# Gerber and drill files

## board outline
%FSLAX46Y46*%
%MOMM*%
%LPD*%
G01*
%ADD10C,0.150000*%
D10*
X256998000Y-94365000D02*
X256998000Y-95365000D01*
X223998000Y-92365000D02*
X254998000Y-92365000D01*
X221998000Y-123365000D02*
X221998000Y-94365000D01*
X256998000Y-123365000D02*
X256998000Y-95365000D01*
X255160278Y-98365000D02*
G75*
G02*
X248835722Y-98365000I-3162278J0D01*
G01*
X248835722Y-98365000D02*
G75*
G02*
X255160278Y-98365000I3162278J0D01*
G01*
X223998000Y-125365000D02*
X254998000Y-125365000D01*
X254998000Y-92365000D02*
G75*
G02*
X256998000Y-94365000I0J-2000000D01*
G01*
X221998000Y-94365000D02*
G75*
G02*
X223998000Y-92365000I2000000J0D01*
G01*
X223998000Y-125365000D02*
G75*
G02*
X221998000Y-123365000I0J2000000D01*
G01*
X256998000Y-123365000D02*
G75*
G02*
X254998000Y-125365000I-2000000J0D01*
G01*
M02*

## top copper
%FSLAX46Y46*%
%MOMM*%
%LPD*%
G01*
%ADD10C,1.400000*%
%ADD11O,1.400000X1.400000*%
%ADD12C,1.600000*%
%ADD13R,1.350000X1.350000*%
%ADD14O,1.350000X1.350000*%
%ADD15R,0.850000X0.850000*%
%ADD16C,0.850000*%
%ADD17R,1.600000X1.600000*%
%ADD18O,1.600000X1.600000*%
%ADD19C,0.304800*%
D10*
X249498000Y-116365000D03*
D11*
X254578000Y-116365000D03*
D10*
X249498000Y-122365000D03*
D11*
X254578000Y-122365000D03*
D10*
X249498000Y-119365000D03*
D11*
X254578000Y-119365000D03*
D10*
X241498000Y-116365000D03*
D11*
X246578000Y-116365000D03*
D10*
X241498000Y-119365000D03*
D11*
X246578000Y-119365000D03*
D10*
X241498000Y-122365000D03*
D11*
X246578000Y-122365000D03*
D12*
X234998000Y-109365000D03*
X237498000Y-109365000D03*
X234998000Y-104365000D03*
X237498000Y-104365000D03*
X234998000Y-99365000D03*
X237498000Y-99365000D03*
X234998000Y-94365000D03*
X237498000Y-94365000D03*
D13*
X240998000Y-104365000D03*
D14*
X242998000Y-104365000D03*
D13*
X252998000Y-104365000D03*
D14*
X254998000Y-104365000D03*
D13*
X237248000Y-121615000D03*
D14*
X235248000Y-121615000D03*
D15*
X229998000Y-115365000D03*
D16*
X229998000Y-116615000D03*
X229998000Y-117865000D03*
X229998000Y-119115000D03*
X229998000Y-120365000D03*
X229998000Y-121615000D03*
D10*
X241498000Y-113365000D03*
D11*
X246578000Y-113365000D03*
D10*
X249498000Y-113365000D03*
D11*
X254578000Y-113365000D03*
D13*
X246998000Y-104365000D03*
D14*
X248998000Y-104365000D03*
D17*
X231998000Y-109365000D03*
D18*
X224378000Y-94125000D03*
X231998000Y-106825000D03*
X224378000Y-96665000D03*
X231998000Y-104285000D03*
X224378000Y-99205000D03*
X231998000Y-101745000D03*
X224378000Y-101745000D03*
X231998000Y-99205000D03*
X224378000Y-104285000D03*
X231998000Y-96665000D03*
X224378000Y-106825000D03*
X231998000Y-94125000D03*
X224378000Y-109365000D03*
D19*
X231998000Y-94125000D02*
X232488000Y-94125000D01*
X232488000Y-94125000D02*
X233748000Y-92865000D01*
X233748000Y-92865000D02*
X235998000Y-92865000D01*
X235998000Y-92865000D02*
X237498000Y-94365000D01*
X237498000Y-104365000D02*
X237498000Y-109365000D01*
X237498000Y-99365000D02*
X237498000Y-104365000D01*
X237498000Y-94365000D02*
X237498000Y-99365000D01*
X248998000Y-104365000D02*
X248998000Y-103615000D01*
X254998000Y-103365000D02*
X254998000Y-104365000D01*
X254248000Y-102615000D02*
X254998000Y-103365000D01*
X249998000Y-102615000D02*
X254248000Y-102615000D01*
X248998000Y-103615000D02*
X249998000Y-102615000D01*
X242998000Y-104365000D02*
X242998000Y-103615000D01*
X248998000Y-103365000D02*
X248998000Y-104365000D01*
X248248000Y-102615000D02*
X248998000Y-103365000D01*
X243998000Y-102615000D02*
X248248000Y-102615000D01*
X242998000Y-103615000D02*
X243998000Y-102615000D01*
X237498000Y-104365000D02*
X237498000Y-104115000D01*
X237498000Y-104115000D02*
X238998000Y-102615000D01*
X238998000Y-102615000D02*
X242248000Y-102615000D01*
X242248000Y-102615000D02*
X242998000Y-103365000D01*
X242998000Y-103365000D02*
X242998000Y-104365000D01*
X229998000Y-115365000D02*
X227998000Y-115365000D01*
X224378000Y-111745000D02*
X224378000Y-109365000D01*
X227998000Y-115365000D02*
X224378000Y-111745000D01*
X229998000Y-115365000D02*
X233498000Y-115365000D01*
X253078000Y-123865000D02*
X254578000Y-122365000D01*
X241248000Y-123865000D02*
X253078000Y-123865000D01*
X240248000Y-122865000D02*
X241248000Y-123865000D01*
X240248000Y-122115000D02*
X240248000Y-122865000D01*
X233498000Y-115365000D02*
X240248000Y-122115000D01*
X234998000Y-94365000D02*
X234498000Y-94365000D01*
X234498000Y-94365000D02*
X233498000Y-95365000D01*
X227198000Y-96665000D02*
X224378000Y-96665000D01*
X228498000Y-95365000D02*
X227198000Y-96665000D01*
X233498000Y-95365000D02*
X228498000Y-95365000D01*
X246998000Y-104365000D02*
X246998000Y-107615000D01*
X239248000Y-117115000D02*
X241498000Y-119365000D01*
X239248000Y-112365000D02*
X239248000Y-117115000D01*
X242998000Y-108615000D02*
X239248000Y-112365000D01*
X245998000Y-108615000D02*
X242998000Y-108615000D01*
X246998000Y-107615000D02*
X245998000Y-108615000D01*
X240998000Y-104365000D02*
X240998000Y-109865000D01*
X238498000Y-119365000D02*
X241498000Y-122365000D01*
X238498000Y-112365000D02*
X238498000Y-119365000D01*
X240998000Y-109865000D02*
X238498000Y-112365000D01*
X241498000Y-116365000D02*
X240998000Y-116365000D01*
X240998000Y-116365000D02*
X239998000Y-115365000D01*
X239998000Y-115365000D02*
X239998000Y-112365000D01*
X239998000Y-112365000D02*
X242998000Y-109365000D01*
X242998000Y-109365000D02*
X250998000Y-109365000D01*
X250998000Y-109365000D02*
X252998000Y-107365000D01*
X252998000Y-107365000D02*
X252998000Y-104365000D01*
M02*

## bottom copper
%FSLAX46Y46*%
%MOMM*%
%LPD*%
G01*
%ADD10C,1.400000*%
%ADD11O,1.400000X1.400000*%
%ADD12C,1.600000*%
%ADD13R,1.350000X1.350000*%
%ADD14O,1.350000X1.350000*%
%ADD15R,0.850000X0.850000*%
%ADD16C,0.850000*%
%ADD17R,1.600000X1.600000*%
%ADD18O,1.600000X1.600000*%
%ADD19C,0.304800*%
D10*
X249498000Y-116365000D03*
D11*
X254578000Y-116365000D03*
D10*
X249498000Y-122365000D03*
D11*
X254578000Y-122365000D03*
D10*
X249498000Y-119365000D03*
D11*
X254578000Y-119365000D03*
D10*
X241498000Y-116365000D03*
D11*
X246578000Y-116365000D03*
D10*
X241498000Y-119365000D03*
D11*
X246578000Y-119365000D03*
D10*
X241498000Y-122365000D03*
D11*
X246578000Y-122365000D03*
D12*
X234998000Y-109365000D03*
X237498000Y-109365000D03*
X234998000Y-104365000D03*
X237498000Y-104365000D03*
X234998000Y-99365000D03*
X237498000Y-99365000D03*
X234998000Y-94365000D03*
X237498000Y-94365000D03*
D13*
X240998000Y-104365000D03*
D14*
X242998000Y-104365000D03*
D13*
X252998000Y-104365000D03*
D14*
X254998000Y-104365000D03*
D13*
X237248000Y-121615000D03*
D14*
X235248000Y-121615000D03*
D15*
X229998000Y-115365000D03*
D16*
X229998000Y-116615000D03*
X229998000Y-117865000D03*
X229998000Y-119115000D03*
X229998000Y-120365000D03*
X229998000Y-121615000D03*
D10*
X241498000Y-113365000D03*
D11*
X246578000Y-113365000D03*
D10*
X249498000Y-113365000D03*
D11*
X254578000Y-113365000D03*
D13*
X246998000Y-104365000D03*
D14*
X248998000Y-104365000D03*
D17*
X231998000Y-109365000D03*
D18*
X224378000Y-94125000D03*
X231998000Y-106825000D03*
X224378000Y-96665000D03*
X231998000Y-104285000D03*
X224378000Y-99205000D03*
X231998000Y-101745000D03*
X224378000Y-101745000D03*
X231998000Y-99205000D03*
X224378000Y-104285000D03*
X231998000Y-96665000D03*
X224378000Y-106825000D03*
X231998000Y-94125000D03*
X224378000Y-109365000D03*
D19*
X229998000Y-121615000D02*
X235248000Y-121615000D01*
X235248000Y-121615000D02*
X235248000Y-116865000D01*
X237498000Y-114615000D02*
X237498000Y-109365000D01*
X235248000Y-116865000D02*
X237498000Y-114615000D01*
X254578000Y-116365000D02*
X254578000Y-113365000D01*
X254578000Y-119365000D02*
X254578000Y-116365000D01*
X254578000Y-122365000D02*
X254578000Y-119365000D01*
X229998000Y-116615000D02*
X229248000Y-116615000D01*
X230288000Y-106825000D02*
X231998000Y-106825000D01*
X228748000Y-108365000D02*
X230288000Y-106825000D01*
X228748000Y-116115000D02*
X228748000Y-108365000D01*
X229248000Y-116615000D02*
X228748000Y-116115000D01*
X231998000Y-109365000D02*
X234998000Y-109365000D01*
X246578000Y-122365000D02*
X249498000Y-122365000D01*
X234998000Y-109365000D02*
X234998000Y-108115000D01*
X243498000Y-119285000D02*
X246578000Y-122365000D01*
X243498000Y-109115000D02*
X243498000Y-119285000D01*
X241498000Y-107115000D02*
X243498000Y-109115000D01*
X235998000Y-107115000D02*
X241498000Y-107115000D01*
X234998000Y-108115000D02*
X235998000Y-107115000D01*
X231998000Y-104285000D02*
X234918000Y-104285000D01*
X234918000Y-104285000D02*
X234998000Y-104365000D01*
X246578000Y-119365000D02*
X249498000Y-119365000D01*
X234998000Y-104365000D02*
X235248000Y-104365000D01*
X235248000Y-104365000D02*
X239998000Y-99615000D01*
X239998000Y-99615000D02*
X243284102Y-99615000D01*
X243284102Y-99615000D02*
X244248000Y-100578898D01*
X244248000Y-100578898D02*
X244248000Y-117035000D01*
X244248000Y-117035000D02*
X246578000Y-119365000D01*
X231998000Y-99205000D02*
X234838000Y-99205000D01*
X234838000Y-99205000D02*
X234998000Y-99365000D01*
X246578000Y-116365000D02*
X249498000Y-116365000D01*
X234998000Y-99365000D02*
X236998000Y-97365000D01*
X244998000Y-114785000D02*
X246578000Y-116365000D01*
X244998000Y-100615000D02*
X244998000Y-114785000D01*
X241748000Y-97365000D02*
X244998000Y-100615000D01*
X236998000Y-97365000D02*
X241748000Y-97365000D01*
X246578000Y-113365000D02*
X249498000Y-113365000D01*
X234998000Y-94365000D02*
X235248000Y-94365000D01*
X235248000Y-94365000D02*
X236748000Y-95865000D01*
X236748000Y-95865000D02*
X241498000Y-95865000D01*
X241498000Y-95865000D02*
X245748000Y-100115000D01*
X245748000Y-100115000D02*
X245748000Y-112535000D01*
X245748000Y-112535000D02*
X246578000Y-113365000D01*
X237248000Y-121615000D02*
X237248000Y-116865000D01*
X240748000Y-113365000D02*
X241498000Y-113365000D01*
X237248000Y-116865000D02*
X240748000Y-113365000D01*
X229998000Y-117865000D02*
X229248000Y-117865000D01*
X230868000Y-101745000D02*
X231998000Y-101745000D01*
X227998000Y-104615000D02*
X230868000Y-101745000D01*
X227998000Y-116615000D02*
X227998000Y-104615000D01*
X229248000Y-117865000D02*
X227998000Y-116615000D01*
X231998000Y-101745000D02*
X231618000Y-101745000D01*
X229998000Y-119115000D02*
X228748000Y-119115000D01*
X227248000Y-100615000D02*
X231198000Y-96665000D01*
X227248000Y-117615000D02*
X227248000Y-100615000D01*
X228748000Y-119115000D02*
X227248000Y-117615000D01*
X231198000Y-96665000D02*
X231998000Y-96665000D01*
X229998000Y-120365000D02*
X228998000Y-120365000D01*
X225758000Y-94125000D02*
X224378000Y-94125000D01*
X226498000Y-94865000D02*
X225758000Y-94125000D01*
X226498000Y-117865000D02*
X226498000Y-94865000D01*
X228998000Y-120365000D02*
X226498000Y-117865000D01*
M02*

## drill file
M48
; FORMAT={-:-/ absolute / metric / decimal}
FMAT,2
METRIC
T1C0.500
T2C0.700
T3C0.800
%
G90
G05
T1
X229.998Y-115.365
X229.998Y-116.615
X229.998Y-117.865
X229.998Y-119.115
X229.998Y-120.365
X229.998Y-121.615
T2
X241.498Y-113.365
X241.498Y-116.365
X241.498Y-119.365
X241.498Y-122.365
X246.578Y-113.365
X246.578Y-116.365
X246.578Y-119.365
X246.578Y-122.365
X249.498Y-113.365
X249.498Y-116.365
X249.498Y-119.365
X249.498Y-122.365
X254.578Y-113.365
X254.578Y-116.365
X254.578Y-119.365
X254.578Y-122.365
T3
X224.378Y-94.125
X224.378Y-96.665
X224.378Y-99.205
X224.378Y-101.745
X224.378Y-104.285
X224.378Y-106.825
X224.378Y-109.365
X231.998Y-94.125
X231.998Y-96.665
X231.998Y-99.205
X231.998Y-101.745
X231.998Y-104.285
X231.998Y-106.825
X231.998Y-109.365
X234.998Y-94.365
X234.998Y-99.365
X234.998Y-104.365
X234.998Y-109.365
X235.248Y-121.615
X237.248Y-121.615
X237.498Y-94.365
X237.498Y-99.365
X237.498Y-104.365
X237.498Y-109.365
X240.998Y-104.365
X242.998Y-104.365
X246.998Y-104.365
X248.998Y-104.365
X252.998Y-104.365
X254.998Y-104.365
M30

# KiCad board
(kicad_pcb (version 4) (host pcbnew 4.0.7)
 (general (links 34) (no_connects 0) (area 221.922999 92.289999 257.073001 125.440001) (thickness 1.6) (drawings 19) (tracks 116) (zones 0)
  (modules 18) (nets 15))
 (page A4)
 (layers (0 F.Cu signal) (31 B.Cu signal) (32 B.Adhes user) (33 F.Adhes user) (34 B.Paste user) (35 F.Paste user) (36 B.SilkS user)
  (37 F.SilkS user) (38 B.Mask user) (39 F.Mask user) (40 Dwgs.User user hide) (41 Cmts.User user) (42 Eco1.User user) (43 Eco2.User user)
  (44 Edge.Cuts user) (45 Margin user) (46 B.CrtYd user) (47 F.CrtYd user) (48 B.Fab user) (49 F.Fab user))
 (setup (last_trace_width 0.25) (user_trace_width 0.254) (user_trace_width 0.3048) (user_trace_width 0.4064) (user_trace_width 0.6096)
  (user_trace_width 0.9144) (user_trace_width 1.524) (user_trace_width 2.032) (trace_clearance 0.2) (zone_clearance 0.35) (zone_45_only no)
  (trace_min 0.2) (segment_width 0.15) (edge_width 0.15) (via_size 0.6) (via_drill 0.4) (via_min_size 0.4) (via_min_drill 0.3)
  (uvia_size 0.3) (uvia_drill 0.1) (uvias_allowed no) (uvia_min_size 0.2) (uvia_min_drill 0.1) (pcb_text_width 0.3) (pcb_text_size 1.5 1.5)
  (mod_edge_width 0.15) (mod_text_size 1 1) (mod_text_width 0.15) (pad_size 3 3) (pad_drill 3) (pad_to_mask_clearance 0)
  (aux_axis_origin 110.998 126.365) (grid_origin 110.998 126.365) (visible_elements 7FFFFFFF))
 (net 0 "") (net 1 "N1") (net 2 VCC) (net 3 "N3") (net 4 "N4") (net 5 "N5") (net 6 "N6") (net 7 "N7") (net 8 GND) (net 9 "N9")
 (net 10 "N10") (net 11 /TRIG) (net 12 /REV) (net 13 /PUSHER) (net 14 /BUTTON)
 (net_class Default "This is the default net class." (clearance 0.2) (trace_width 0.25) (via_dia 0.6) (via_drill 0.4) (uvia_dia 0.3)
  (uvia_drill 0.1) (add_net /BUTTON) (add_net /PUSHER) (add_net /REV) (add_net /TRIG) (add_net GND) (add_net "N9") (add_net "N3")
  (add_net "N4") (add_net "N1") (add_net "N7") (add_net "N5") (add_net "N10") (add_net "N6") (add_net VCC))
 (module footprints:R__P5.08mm (layer F.Cu) (at 251.998 116.365)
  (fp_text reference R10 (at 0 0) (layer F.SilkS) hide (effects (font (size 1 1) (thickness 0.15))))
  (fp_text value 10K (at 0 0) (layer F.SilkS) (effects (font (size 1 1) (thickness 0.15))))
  (pad 1 thru_hole circle (at -2.5 0) (size 1.4 1.4) (drill 0.7) (layers *.Cu *.Mask) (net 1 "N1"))
  (pad 2 thru_hole oval (at 2.58 0) (size 1.4 1.4) (drill 0.7) (layers *.Cu *.Mask) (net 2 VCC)))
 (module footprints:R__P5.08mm (layer F.Cu) (at 251.998 122.365)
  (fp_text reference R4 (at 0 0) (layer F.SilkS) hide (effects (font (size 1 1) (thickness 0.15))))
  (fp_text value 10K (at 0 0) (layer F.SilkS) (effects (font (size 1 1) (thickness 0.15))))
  (pad 1 thru_hole circle (at -2.5 0) (size 1.4 1.4) (drill 0.7) (layers *.Cu *.Mask) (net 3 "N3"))
  (pad 2 thru_hole oval (at 2.58 0) (size 1.4 1.4) (drill 0.7) (layers *.Cu *.Mask) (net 2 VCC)))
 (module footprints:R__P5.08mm (layer F.Cu) (at 251.998 119.365)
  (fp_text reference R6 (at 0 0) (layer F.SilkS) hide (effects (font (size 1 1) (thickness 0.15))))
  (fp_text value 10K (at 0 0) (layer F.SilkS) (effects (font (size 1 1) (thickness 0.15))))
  (pad 1 thru_hole circle (at -2.5 0) (size 1.4 1.4) (drill 0.7) (layers *.Cu *.Mask) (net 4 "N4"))
  (pad 2 thru_hole oval (at 2.58 0) (size 1.4 1.4) (drill 0.7) (layers *.Cu *.Mask) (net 2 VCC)))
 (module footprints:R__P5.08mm (layer F.Cu) (at 243.998 116.365)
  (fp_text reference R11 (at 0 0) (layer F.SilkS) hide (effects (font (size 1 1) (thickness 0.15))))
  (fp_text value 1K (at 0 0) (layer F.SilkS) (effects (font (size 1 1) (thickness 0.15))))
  (pad 1 thru_hole circle (at -2.5 0) (size 1.4 1.4) (drill 0.7) (layers *.Cu *.Mask) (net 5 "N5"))
  (pad 2 thru_hole oval (at 2.58 0) (size 1.4 1.4) (drill 0.7) (layers *.Cu *.Mask) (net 1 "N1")))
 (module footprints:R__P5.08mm (layer F.Cu) (at 243.998 119.365)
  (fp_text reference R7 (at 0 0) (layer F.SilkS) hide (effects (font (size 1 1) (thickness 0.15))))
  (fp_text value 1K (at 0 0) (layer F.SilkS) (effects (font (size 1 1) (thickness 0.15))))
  (pad 1 thru_hole circle (at -2.5 0) (size 1.4 1.4) (drill 0.7) (layers *.Cu *.Mask) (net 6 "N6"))
  (pad 2 thru_hole oval (at 2.58 0) (size 1.4 1.4) (drill 0.7) (layers *.Cu *.Mask) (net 4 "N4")))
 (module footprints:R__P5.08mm (layer F.Cu) (at 243.998 122.365)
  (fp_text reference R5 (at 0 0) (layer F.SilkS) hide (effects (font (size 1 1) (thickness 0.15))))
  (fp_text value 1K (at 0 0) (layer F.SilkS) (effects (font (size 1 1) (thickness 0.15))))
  (pad 1 thru_hole circle (at -2.5 0) (size 1.4 1.4) (drill 0.7) (layers *.Cu *.Mask) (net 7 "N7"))
  (pad 2 thru_hole oval (at 2.58 0) (size 1.4 1.4) (drill 0.7) (layers *.Cu *.Mask) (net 3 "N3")))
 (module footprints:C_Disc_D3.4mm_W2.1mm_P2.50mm (layer F.Cu) (at 234.998 109.365)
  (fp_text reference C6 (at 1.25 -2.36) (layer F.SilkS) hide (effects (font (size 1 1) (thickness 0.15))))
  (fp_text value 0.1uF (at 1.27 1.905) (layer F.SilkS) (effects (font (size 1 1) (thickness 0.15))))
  (pad 1 thru_hole circle (at 0 0) (size 1.6 1.6) (drill 0.8) (layers *.Cu *.Mask) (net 3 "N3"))
  (pad 2 thru_hole circle (at 2.5 0) (size 1.6 1.6) (drill 0.8) (layers *.Cu *.Mask) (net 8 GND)))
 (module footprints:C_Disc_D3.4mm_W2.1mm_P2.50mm (layer F.Cu) (at 234.998 104.365)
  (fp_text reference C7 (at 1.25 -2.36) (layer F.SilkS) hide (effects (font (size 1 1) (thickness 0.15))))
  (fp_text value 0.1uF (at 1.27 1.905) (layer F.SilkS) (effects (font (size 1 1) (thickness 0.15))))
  (pad 1 thru_hole circle (at 0 0) (size 1.6 1.6) (drill 0.8) (layers *.Cu *.Mask) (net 4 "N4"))
  (pad 2 thru_hole circle (at 2.5 0) (size 1.6 1.6) (drill 0.8) (layers *.Cu *.Mask) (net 8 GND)))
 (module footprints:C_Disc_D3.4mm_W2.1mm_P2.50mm (layer F.Cu) (at 234.998 99.365)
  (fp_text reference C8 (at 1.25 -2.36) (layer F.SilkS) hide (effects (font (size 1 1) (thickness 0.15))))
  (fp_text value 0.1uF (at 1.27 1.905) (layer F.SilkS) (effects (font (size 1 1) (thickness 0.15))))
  (pad 1 thru_hole circle (at 0 0) (size 1.6 1.6) (drill 0.8) (layers *.Cu *.Mask) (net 1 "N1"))
  (pad 2 thru_hole circle (at 2.5 0) (size 1.6 1.6) (drill 0.8) (layers *.Cu *.Mask) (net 8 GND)))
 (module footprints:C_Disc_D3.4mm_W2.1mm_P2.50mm (layer F.Cu) (at 234.998 94.365)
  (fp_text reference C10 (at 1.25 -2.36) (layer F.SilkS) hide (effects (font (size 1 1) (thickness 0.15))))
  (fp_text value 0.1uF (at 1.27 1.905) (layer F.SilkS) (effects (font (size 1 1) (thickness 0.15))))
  (pad 1 thru_hole circle (at 0 0) (size 1.6 1.6) (drill 0.8) (layers *.Cu *.Mask) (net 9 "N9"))
  (pad 2 thru_hole circle (at 2.5 0) (size 1.6 1.6) (drill 0.8) (layers *.Cu *.Mask) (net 8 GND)))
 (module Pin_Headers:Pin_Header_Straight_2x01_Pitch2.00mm (layer F.Cu) (at 240.998 104.365)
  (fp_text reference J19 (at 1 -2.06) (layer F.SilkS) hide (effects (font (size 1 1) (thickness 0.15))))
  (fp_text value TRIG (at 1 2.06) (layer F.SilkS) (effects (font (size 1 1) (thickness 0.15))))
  (pad 1 thru_hole rect (at 0 0) (size 1.35 1.35) (drill 0.8) (layers *.Cu *.Mask) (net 7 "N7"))
  (pad 2 thru_hole oval (at 2 0) (size 1.35 1.35) (drill 0.8) (layers *.Cu *.Mask) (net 8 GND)))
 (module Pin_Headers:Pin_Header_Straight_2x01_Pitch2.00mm (layer F.Cu) (at 252.998 104.365)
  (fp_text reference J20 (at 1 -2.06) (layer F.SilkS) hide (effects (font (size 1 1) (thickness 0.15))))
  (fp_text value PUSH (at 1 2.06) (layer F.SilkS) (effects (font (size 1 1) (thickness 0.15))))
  (pad 1 thru_hole rect (at 0 0) (size 1.35 1.35) (drill 0.8) (layers *.Cu *.Mask) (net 5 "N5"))
  (pad 2 thru_hole oval (at 2 0) (size 1.35 1.35) (drill 0.8) (layers *.Cu *.Mask) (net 8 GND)))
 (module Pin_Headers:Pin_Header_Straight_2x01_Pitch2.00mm (layer F.Cu) (at 237.248 121.615 180)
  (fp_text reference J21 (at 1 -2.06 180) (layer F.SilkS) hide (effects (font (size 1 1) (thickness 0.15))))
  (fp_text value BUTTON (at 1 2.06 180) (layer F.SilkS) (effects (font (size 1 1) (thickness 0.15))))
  (pad 1 thru_hole rect (at 0 0 180) (size 1.35 1.35) (drill 0.8) (layers *.Cu *.Mask) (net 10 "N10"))
  (pad 2 thru_hole oval (at 2 0 180) (size 1.35 1.35) (drill 0.8) (layers *.Cu *.Mask) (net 8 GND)))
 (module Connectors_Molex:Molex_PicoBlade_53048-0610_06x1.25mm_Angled (layer F.Cu) (at 229.998 115.365 270)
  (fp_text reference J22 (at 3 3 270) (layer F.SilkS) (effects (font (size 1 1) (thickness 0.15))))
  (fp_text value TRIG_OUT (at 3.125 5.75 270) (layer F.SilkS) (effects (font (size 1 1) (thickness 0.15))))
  (pad 1 thru_hole rect (at 0 0 270) (size 0.85 0.85) (drill 0.5) (layers *.Cu *.Mask) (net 2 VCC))
  (pad 2 thru_hole circle (at 1.25 0 270) (size 0.85 0.85) (drill 0.5) (layers *.Cu *.Mask) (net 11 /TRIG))
  (pad 3 thru_hole circle (at 2.5 0 270) (size 0.85 0.85) (drill 0.5) (layers *.Cu *.Mask) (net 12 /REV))
  (pad 4 thru_hole circle (at 3.75 0 270) (size 0.85 0.85) (drill 0.5) (layers *.Cu *.Mask) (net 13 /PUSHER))
  (pad 5 thru_hole circle (at 5 0 270) (size 0.85 0.85) (drill 0.5) (layers *.Cu *.Mask) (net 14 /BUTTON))
  (pad 6 thru_hole circle (at 6.25 0 270) (size 0.85 0.85) (drill 0.5) (layers *.Cu *.Mask) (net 8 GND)))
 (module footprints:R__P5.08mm (layer F.Cu) (at 243.998 113.365)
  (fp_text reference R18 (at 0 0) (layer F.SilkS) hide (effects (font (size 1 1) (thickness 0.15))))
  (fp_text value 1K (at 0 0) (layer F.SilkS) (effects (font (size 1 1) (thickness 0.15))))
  (pad 1 thru_hole circle (at -2.5 0) (size 1.4 1.4) (drill 0.7) (layers *.Cu *.Mask) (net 10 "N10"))
  (pad 2 thru_hole oval (at 2.58 0) (size 1.4 1.4) (drill 0.7) (layers *.Cu *.Mask) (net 9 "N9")))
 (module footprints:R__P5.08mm (layer F.Cu) (at 251.998 113.365)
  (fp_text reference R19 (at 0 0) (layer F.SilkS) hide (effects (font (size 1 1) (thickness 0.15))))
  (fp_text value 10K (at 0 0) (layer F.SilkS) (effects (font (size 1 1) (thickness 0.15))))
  (pad 1 thru_hole circle (at -2.5 0) (size 1.4 1.4) (drill 0.7) (layers *.Cu *.Mask) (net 9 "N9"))
  (pad 2 thru_hole oval (at 2.58 0) (size 1.4 1.4) (drill 0.7) (layers *.Cu *.Mask) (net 2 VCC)))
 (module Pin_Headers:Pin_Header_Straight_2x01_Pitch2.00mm (layer F.Cu) (at 246.998 104.365)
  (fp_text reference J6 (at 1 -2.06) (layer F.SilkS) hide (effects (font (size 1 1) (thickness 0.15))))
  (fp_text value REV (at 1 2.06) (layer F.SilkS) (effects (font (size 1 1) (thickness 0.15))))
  (pad 1 thru_hole rect (at 0 0) (size 1.35 1.35) (drill 0.8) (layers *.Cu *.Mask) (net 6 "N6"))
  (pad 2 thru_hole oval (at 2 0) (size 1.35 1.35) (drill 0.8) (layers *.Cu *.Mask) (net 8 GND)))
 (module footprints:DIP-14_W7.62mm (layer F.Cu) (at 231.998 109.365 180)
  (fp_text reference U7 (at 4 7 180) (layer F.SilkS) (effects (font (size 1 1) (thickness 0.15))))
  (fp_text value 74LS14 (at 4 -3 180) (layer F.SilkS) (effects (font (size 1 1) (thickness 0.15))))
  (pad 1 thru_hole rect (at 0 0 180) (size 1.6 1.6) (drill 0.8) (layers *.Cu *.Mask) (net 3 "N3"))
  (pad 8 thru_hole oval (at 7.62 15.24 180) (size 1.6 1.6) (drill 0.8) (layers *.Cu *.Mask) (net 14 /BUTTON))
  (pad 2 thru_hole oval (at 0 2.54 180) (size 1.6 1.6) (drill 0.8) (layers *.Cu *.Mask) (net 11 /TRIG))
  (pad 9 thru_hole oval (at 7.62 12.7 180) (size 1.6 1.6) (drill 0.8) (layers *.Cu *.Mask) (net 9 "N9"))
  (pad 3 thru_hole oval (at 0 5.08 180) (size 1.6 1.6) (drill 0.8) (layers *.Cu *.Mask) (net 4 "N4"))
  (pad 10 thru_hole oval (at 7.62 10.16 180) (size 1.6 1.6) (drill 0.8) (layers *.Cu *.Mask))
  (pad 4 thru_hole oval (at 0 7.62 180) (size 1.6 1.6) (drill 0.8) (layers *.Cu *.Mask) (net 12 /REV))
  (pad 11 thru_hole oval (at 7.62 7.62 180) (size 1.6 1.6) (drill 0.8) (layers *.Cu *.Mask))
  (pad 5 thru_hole oval (at 0 10.16 180) (size 1.6 1.6) (drill 0.8) (layers *.Cu *.Mask) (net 1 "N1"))
  (pad 12 thru_hole oval (at 7.62 5.08 180) (size 1.6 1.6) (drill 0.8) (layers *.Cu *.Mask))
  (pad 6 thru_hole oval (at 0 12.7 180) (size 1.6 1.6) (drill 0.8) (layers *.Cu *.Mask) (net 13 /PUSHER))
  (pad 13 thru_hole oval (at 7.62 2.54 180) (size 1.6 1.6) (drill 0.8) (layers *.Cu *.Mask))
  (pad 7 thru_hole oval (at 0 15.24 180) (size 1.6 1.6) (drill 0.8) (layers *.Cu *.Mask) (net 8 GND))
  (pad 14 thru_hole oval (at 7.62 0 180) (size 1.6 1.6) (drill 0.8) (layers *.Cu *.Mask) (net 2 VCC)))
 (gr_line (start 256.998 94.365) (end 256.998 95.365) (angle 90) (layer Edge.Cuts) (width 0.15))
 (gr_line (start 223.998 92.365) (end 254.998 92.365) (angle 90) (layer Edge.Cuts) (width 0.15))
 (gr_line (start 221.998 123.365) (end 221.998 94.365) (angle 90) (layer Edge.Cuts) (width 0.15))
 (gr_line (start 256.998 123.365) (end 256.998 95.365) (angle 90) (layer Edge.Cuts) (width 0.15))
 (gr_circle (center 251.998 98.365) (end 252.998 95.365) (layer Edge.Cuts) (width 0.15))
 (gr_line (start 223.998 125.365) (end 254.998 125.365) (angle 90) (layer Edge.Cuts) (width 0.15))
 (gr_arc (start 254.998 94.365) (end 254.998 92.365) (angle 90) (layer Edge.Cuts) (width 0.15))
 (gr_arc (start 223.998 94.365) (end 221.998 94.365) (angle 90) (layer Edge.Cuts) (width 0.15))
 (gr_arc (start 223.998 123.365) (end 223.998 125.365) (angle 90) (layer Edge.Cuts) (width 0.15))
 (gr_arc (start 254.998 123.365) (end 256.998 123.365) (angle 90) (layer Edge.Cuts) (width 0.15))
 (segment (start 231.998 94.125) (end 232.488 94.125) (width 0.3048) (layer F.Cu) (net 8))
 (segment (start 232.488 94.125) (end 233.748 92.865) (width 0.3048) (layer F.Cu) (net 8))
 (segment (start 233.748 92.865) (end 235.998 92.865) (width 0.3048) (layer F.Cu) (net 8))
 (segment (start 235.998 92.865) (end 237.498 94.365) (width 0.3048) (layer F.Cu) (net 8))
 (segment (start 229.998 121.615) (end 235.248 121.615) (width 0.3048) (layer B.Cu) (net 8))
 (segment (start 235.248 121.615) (end 235.248 116.865) (width 0.3048) (layer B.Cu) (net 8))
 (segment (start 237.498 114.615) (end 237.498 109.365) (width 0.3048) (layer B.Cu) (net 8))
 (segment (start 235.248 116.865) (end 237.498 114.615) (width 0.3048) (layer B.Cu) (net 8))
 (segment (start 237.498 104.365) (end 237.498 109.365) (width 0.3048) (layer F.Cu) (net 8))
 (segment (start 237.498 99.365) (end 237.498 104.365) (width 0.3048) (layer F.Cu) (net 8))
 (segment (start 237.498 94.365) (end 237.498 99.365) (width 0.3048) (layer F.Cu) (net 8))
 (segment (start 248.998 104.365) (end 248.998 103.615) (width 0.3048) (layer F.Cu) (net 8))
 (segment (start 254.998 103.365) (end 254.998 104.365) (width 0.3048) (layer F.Cu) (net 8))
 (segment (start 254.248 102.615) (end 254.998 103.365) (width 0.3048) (layer F.Cu) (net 8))
 (segment (start 249.998 102.615) (end 254.248 102.615) (width 0.3048) (layer F.Cu) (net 8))
 (segment (start 248.998 103.615) (end 249.998 102.615) (width 0.3048) (layer F.Cu) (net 8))
 (segment (start 242.998 104.365) (end 242.998 103.615) (width 0.3048) (layer F.Cu) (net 8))
 (segment (start 248.998 103.365) (end 248.998 104.365) (width 0.3048) (layer F.Cu) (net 8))
 (segment (start 248.248 102.615) (end 248.998 103.365) (width 0.3048) (layer F.Cu) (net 8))
 (segment (start 243.998 102.615) (end 248.248 102.615) (width 0.3048) (layer F.Cu) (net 8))
 (segment (start 242.998 103.615) (end 243.998 102.615) (width 0.3048) (layer F.Cu) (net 8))
 (segment (start 237.498 104.365) (end 237.498 104.115) (width 0.3048) (layer F.Cu) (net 8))
 (segment (start 237.498 104.115) (end 238.998 102.615) (width 0.3048) (layer F.Cu) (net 8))
 (segment (start 238.998 102.615) (end 242.248 102.615) (width 0.3048) (layer F.Cu) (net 8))
 (segment (start 242.248 102.615) (end 242.998 103.365) (width 0.3048) (layer F.Cu) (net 8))
 (segment (start 242.998 103.365) (end 242.998 104.365) (width 0.3048) (layer F.Cu) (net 8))
 (segment (start 229.998 115.365) (end 227.998 115.365) (width 0.3048) (layer F.Cu) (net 2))
 (segment (start 224.378 111.745) (end 224.378 109.365) (width 0.3048) (layer F.Cu) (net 2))
 (segment (start 227.998 115.365) (end 224.378 111.745) (width 0.3048) (layer F.Cu) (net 2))
 (segment (start 229.998 115.365) (end 233.498 115.365) (width 0.3048) (layer F.Cu) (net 2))
 (segment (start 253.078 123.865) (end 254.578 122.365) (width 0.3048) (layer F.Cu) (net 2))
 (segment (start 241.248 123.865) (end 253.078 123.865) (width 0.3048) (layer F.Cu) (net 2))
 (segment (start 240.248 122.865) (end 241.248 123.865) (width 0.3048) (layer F.Cu) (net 2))
 (segment (start 240.248 122.115) (end 240.248 122.865) (width 0.3048) (layer F.Cu) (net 2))
 (segment (start 233.498 115.365) (end 240.248 122.115) (width 0.3048) (layer F.Cu) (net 2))
 (segment (start 254.578 116.365) (end 254.578 113.365) (width 0.3048) (layer B.Cu) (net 2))
 (segment (start 254.578 119.365) (end 254.578 116.365) (width 0.3048) (layer B.Cu) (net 2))
 (segment (start 254.578 122.365) (end 254.578 119.365) (width 0.3048) (layer B.Cu) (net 2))
 (segment (start 229.998 116.615) (end 229.248 116.615) (width 0.3048) (layer B.Cu) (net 11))
 (segment (start 230.288 106.825) (end 231.998 106.825) (width 0.3048) (layer B.Cu) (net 11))
 (segment (start 228.748 108.365) (end 230.288 106.825) (width 0.3048) (layer B.Cu) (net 11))
 (segment (start 228.748 116.115) (end 228.748 108.365) (width 0.3048) (layer B.Cu) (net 11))
 (segment (start 229.248 116.615) (end 228.748 116.115) (width 0.3048) (layer B.Cu) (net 11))
 (segment (start 231.998 109.365) (end 234.998 109.365) (width 0.3048) (layer B.Cu) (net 3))
 (segment (start 246.578 122.365) (end 249.498 122.365) (width 0.3048) (layer B.Cu) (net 3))
 (segment (start 234.998 109.365) (end 234.998 108.115) (width 0.3048) (layer B.Cu) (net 3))
 (segment (start 243.498 119.285) (end 246.578 122.365) (width 0.3048) (layer B.Cu) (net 3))
 (segment (start 243.498 109.115) (end 243.498 119.285) (width 0.3048) (layer B.Cu) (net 3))
 (segment (start 241.498 107.115) (end 243.498 109.115) (width 0.3048) (layer B.Cu) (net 3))
 (segment (start 235.998 107.115) (end 241.498 107.115) (width 0.3048) (layer B.Cu) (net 3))
 (segment (start 234.998 108.115) (end 235.998 107.115) (width 0.3048) (layer B.Cu) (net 3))
 (segment (start 231.998 104.285) (end 234.918 104.285) (width 0.3048) (layer B.Cu) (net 4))
 (segment (start 234.918 104.285) (end 234.998 104.365) (width 0.3048) (layer B.Cu) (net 4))
 (segment (start 246.578 119.365) (end 249.498 119.365) (width 0.3048) (layer B.Cu) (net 4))
 (segment (start 234.998 104.365) (end 235.248 104.365) (width 0.3048) (layer B.Cu) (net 4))
 (segment (start 235.248 104.365) (end 239.998 99.615) (width 0.3048) (layer B.Cu) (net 4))
 (segment (start 239.998 99.615) (end 243.284102 99.615) (width 0.3048) (layer B.Cu) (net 4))
 (segment (start 243.284102 99.615) (end 244.248 100.578898) (width 0.3048) (layer B.Cu) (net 4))
 (segment (start 244.248 100.578898) (end 244.248 117.035) (width 0.3048) (layer B.Cu) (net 4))
 (segment (start 244.248 117.035) (end 246.578 119.365) (width 0.3048) (layer B.Cu) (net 4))
 (segment (start 231.998 99.205) (end 234.838 99.205) (width 0.3048) (layer B.Cu) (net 1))
 (segment (start 234.838 99.205) (end 234.998 99.365) (width 0.3048) (layer B.Cu) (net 1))
 (segment (start 246.578 116.365) (end 249.498 116.365) (width 0.3048) (layer B.Cu) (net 1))
 (segment (start 234.998 99.365) (end 236.998 97.365) (width 0.3048) (layer B.Cu) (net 1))
 (segment (start 244.998 114.785) (end 246.578 116.365) (width 0.3048) (layer B.Cu) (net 1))
 (segment (start 244.998 100.615) (end 244.998 114.785) (width 0.3048) (layer B.Cu) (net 1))
 (segment (start 241.748 97.365) (end 244.998 100.615) (width 0.3048) (layer B.Cu) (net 1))
 (segment (start 236.998 97.365) (end 241.748 97.365) (width 0.3048) (layer B.Cu) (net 1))
 (segment (start 234.998 94.365) (end 234.498 94.365) (width 0.3048) (layer F.Cu) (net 9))
 (segment (start 234.498 94.365) (end 233.498 95.365) (width 0.3048) (layer F.Cu) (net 9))
 (segment (start 227.198 96.665) (end 224.378 96.665) (width 0.3048) (layer F.Cu) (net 9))
 (segment (start 228.498 95.365) (end 227.198 96.665) (width 0.3048) (layer F.Cu) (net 9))
 (segment (start 233.498 95.365) (end 228.498 95.365) (width 0.3048) (layer F.Cu) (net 9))
 (segment (start 246.578 113.365) (end 249.498 113.365) (width 0.3048) (layer B.Cu) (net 9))
 (segment (start 234.998 94.365) (end 235.248 94.365) (width 0.3048) (layer B.Cu) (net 9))
 (segment (start 235.248 94.365) (end 236.748 95.865) (width 0.3048) (layer B.Cu) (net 9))
 (segment (start 236.748 95.865) (end 241.498 95.865) (width 0.3048) (layer B.Cu) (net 9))
 (segment (start 241.498 95.865) (end 245.748 100.115) (width 0.3048) (layer B.Cu) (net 9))
 (segment (start 245.748 100.115) (end 245.748 112.535) (width 0.3048) (layer B.Cu) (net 9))
 (segment (start 245.748 112.535) (end 246.578 113.365) (width 0.3048) (layer B.Cu) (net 9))
 (segment (start 246.998 104.365) (end 246.998 107.615) (width 0.3048) (layer F.Cu) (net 6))
 (segment (start 239.248 117.115) (end 241.498 119.365) (width 0.3048) (layer F.Cu) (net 6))
 (segment (start 239.248 112.365) (end 239.248 117.115) (width 0.3048) (layer F.Cu) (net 6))
 (segment (start 242.998 108.615) (end 239.248 112.365) (width 0.3048) (layer F.Cu) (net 6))
 (segment (start 245.998 108.615) (end 242.998 108.615) (width 0.3048) (layer F.Cu) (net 6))
 (segment (start 246.998 107.615) (end 245.998 108.615) (width 0.3048) (layer F.Cu) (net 6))
 (segment (start 240.998 104.365) (end 240.998 109.865) (width 0.3048) (layer F.Cu) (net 7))
 (segment (start 238.498 119.365) (end 241.498 122.365) (width 0.3048) (layer F.Cu) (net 7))
 (segment (start 238.498 112.365) (end 238.498 119.365) (width 0.3048) (layer F.Cu) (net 7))
 (segment (start 240.998 109.865) (end 238.498 112.365) (width 0.3048) (layer F.Cu) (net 7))
 (segment (start 241.498 116.365) (end 240.998 116.365) (width 0.3048) (layer F.Cu) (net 5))
 (segment (start 240.998 116.365) (end 239.998 115.365) (width 0.3048) (layer F.Cu) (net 5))
 (segment (start 239.998 115.365) (end 239.998 112.365) (width 0.3048) (layer F.Cu) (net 5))
 (segment (start 239.998 112.365) (end 242.998 109.365) (width 0.3048) (layer F.Cu) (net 5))
 (segment (start 242.998 109.365) (end 250.998 109.365) (width 0.3048) (layer F.Cu) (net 5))
 (segment (start 250.998 109.365) (end 252.998 107.365) (width 0.3048) (layer F.Cu) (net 5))
 (segment (start 252.998 107.365) (end 252.998 104.365) (width 0.3048) (layer F.Cu) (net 5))
 (segment (start 237.248 121.615) (end 237.248 116.865) (width 0.3048) (layer B.Cu) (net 10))
 (segment (start 240.748 113.365) (end 241.498 113.365) (width 0.3048) (layer B.Cu) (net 10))
 (segment (start 237.248 116.865) (end 240.748 113.365) (width 0.3048) (layer B.Cu) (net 10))
 (segment (start 229.998 117.865) (end 229.248 117.865) (width 0.3048) (layer B.Cu) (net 12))
 (segment (start 230.868 101.745) (end 231.998 101.745) (width 0.3048) (layer B.Cu) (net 12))
 (segment (start 227.998 104.615) (end 230.868 101.745) (width 0.3048) (layer B.Cu) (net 12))
 (segment (start 227.998 116.615) (end 227.998 104.615) (width 0.3048) (layer B.Cu) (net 12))
 (segment (start 229.248 117.865) (end 227.998 116.615) (width 0.3048) (layer B.Cu) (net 12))
 (segment (start 231.998 101.745) (end 231.618 101.745) (width 0.3048) (layer B.Cu) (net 12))
 (segment (start 229.998 119.115) (end 228.748 119.115) (width 0.3048) (layer B.Cu) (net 13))
 (segment (start 227.248 100.615) (end 231.198 96.665) (width 0.3048) (layer B.Cu) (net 13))
 (segment (start 227.248 117.615) (end 227.248 100.615) (width 0.3048) (layer B.Cu) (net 13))
 (segment (start 228.748 119.115) (end 227.248 117.615) (width 0.3048) (layer B.Cu) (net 13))
 (segment (start 231.198 96.665) (end 231.998 96.665) (width 0.3048) (layer B.Cu) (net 13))
 (segment (start 229.998 120.365) (end 228.998 120.365) (width 0.3048) (layer B.Cu) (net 14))
 (segment (start 225.758 94.125) (end 224.378 94.125) (width 0.3048) (layer B.Cu) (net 14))
 (segment (start 226.498 94.865) (end 225.758 94.125) (width 0.3048) (layer B.Cu) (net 14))
 (segment (start 226.498 117.865) (end 226.498 94.865) (width 0.3048) (layer B.Cu) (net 14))
 (segment (start 228.998 120.365) (end 226.498 117.865) (width 0.3048) (layer B.Cu) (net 14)))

